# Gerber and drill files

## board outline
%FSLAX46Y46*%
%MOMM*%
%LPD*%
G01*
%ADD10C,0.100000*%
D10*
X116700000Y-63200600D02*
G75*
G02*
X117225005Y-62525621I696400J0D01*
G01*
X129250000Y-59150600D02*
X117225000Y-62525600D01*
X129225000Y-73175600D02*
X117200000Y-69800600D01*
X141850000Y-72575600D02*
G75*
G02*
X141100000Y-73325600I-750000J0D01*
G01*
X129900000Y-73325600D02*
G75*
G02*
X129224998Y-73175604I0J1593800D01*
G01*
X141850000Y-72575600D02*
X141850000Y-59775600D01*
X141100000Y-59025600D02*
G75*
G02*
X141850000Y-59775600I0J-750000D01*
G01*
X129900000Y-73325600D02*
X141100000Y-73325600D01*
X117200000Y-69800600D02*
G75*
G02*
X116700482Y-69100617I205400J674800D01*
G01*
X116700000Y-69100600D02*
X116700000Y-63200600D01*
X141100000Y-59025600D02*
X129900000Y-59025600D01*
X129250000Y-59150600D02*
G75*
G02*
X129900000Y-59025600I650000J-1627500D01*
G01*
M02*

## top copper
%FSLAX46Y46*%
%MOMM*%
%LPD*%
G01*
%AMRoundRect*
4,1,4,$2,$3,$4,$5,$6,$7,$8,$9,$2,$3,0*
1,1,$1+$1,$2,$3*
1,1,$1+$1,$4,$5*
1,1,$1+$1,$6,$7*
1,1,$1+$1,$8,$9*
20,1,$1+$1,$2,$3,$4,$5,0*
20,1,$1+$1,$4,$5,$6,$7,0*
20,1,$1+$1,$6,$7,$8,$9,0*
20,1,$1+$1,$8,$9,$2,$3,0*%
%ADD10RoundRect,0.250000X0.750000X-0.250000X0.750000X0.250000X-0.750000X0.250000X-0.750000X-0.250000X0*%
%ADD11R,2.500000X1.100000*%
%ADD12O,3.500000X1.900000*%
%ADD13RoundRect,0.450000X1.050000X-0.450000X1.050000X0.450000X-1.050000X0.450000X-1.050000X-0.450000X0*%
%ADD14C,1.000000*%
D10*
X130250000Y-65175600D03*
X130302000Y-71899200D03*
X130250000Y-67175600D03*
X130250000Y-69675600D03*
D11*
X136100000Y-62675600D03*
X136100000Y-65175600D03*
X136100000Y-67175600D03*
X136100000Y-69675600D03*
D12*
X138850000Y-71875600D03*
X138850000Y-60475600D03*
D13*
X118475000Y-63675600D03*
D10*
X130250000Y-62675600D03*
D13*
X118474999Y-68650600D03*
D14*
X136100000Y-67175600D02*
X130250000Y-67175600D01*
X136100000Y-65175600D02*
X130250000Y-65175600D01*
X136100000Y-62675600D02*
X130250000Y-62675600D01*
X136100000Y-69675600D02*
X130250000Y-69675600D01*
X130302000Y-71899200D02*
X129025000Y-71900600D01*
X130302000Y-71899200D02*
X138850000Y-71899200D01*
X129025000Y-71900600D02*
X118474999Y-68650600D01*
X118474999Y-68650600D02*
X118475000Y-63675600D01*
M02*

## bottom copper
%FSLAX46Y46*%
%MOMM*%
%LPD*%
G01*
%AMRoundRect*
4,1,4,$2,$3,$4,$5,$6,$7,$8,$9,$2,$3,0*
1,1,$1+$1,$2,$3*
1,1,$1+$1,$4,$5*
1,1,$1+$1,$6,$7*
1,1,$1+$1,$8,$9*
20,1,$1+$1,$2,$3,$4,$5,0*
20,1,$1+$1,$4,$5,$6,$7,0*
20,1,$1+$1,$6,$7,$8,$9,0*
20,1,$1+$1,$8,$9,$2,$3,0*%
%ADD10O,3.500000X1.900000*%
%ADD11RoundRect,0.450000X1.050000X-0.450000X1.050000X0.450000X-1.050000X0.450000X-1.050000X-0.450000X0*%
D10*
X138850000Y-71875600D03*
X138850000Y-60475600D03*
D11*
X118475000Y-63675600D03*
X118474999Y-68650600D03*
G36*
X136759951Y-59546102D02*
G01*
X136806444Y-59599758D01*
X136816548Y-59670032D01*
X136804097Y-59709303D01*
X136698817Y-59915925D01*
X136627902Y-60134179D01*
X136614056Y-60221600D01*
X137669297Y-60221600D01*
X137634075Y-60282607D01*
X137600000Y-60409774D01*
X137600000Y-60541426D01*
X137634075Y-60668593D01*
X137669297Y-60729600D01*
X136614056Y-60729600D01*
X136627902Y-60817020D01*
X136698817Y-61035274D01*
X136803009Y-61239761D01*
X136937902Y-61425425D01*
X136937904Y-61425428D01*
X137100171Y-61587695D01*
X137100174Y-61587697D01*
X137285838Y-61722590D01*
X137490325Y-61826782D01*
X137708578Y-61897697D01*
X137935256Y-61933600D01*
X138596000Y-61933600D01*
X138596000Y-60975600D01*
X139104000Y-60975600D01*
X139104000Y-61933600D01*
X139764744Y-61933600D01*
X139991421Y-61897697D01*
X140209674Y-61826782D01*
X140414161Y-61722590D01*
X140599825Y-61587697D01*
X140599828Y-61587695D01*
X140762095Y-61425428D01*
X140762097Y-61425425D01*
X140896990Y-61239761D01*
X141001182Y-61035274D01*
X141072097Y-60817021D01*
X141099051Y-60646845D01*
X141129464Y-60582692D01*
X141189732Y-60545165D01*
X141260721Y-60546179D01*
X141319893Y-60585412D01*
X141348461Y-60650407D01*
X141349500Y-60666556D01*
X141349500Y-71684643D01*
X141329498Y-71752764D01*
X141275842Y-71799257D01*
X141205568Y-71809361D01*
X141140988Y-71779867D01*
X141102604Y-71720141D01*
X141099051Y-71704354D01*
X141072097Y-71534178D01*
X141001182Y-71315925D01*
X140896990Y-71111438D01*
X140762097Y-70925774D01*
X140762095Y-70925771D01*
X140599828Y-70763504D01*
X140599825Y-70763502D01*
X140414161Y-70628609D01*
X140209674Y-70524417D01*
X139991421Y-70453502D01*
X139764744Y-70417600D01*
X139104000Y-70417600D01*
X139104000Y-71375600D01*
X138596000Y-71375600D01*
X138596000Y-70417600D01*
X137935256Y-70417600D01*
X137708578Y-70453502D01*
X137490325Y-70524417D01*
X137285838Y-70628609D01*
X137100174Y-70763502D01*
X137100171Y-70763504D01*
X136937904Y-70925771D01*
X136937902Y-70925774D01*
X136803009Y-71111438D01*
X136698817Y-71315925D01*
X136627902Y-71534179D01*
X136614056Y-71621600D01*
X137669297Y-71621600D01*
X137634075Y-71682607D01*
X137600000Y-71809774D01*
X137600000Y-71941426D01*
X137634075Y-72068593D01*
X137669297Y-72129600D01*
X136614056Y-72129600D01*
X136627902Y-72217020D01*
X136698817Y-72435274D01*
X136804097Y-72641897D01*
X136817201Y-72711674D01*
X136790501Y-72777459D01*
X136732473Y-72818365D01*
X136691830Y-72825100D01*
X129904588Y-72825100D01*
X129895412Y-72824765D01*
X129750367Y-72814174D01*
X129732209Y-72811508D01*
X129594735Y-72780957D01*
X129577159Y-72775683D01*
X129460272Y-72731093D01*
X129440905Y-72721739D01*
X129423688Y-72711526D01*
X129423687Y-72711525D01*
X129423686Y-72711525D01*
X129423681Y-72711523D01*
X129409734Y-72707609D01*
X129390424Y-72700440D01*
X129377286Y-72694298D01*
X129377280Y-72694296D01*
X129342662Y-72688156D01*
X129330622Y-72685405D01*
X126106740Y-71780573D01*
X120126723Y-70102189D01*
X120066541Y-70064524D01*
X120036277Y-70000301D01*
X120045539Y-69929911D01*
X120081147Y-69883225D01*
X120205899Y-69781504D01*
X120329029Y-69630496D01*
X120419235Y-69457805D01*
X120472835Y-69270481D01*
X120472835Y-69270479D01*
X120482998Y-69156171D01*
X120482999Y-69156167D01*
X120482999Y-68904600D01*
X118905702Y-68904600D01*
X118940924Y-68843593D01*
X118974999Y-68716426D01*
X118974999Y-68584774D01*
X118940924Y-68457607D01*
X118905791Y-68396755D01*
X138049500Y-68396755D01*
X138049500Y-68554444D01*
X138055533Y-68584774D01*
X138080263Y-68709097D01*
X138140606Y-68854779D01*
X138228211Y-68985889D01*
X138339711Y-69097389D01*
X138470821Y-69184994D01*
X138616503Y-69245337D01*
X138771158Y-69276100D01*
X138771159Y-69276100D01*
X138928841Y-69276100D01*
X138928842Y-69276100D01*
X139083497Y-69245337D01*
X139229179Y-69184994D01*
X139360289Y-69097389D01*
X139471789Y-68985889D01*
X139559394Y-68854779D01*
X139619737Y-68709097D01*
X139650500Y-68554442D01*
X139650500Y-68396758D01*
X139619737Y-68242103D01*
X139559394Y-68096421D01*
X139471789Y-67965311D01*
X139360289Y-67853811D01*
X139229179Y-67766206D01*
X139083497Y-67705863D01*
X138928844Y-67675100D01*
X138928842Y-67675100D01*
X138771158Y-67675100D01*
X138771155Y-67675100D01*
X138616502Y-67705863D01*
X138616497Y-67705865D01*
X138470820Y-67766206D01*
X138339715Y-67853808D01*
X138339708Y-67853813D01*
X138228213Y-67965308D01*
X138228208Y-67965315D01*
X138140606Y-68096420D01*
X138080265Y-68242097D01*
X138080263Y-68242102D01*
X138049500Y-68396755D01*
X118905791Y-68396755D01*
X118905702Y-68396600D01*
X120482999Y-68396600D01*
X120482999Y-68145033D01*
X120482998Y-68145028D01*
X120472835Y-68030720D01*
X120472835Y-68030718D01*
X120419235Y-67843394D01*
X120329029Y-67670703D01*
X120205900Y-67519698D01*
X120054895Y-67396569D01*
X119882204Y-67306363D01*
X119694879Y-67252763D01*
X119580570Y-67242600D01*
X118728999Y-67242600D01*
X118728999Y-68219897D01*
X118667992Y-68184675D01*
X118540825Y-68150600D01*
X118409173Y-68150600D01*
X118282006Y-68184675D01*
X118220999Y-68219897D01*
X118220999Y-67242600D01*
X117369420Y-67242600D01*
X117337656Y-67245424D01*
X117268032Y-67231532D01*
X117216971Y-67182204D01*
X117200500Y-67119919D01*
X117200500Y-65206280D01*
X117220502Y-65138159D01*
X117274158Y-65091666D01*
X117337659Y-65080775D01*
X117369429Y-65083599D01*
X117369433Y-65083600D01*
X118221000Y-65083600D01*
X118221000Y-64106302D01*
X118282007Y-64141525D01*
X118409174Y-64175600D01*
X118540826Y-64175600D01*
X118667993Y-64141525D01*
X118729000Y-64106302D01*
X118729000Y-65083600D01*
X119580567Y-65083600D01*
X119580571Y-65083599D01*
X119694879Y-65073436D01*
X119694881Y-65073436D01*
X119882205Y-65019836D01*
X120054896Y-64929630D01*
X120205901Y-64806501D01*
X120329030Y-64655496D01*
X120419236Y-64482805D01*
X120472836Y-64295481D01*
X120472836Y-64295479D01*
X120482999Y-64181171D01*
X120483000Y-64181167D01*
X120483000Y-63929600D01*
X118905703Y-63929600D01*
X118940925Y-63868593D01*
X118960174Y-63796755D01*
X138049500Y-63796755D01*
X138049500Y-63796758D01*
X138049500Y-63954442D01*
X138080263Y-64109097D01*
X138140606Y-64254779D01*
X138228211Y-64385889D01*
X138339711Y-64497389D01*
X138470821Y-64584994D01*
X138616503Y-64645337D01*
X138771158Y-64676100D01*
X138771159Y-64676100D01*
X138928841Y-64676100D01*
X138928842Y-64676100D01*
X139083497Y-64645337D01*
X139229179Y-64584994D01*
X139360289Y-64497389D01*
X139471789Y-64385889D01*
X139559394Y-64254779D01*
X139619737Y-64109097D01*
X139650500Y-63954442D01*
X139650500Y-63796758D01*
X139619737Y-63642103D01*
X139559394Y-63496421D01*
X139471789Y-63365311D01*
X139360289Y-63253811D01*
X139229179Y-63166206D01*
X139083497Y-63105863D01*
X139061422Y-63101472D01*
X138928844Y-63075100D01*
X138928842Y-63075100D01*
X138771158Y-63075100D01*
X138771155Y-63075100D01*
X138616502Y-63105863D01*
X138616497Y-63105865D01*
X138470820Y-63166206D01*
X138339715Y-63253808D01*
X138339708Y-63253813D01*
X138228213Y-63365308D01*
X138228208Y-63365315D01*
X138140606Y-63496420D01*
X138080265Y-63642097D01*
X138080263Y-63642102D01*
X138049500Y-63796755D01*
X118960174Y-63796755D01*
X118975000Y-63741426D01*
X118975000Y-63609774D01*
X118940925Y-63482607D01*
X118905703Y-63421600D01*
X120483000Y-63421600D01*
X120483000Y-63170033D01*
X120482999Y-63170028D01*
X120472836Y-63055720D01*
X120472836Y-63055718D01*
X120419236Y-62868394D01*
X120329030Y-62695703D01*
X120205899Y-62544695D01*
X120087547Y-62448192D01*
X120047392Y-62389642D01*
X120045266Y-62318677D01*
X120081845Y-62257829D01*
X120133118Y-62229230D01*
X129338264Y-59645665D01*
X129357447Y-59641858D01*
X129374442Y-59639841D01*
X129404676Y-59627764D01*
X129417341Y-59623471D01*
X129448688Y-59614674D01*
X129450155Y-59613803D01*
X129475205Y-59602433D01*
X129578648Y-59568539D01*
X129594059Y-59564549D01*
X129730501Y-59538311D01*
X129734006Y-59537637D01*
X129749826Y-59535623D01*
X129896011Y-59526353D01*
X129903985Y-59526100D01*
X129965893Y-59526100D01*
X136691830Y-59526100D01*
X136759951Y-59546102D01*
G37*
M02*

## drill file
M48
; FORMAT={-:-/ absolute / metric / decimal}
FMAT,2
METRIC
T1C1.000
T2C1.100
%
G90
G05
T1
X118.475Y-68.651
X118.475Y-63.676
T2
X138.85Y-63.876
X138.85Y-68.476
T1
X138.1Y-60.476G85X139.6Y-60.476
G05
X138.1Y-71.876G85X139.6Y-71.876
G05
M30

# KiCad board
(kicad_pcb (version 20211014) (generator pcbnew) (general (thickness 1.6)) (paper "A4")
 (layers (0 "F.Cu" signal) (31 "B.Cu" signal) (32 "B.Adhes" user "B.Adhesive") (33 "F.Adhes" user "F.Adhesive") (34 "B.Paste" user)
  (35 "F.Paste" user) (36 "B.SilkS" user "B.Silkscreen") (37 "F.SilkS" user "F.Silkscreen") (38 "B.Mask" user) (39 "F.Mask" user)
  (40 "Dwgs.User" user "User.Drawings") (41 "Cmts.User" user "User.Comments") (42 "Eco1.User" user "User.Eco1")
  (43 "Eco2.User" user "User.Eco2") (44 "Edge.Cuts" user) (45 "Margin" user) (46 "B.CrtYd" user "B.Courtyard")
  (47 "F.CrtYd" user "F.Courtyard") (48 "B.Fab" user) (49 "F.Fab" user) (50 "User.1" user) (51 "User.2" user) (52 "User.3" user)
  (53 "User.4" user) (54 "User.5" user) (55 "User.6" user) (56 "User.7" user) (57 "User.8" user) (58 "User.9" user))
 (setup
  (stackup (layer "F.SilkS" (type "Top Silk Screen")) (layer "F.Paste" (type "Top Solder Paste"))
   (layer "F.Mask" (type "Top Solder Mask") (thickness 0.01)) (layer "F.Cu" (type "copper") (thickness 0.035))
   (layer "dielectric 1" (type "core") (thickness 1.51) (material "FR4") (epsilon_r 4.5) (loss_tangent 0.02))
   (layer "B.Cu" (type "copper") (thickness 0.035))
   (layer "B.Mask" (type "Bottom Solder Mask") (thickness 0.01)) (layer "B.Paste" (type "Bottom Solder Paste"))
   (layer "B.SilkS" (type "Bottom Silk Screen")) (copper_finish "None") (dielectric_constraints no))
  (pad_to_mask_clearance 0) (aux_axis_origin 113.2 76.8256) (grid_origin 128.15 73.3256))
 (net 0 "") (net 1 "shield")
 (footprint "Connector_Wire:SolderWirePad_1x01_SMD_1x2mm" (layer "F.Cu") (at 130.25 65.1756 90)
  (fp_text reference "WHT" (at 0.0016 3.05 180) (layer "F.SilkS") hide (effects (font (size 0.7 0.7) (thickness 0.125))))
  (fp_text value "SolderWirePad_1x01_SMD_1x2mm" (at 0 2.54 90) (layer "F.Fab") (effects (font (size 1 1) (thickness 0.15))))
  (pad "1" smd roundrect (at 0 0 90) (size 1 2) (layers "F.Cu" "F.Paste" "F.Mask") (roundrect_rratio 0.25)))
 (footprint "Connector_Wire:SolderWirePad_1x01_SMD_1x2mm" (layer "F.Cu") (at 130.302 71.8992 90)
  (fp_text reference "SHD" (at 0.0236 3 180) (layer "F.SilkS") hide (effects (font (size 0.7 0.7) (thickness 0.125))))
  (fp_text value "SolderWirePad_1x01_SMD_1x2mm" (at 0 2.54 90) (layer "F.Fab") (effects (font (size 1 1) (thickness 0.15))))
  (pad "1" smd roundrect (at 0 0 90) (size 1 2) (layers "F.Cu" "F.Paste" "F.Mask") (roundrect_rratio 0.25)))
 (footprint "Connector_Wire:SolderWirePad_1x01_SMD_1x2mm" (layer "F.Cu") (at 130.25 67.1756 90)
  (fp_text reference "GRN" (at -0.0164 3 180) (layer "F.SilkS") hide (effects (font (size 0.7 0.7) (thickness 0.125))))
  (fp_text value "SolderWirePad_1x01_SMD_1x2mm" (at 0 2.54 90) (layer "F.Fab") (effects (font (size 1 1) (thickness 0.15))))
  (pad "1" smd roundrect (at 0 0 90) (size 1 2) (layers "F.Cu" "F.Paste" "F.Mask") (roundrect_rratio 0.25)))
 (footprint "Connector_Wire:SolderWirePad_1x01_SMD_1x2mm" (layer "F.Cu") (at 130.25 69.6756 90)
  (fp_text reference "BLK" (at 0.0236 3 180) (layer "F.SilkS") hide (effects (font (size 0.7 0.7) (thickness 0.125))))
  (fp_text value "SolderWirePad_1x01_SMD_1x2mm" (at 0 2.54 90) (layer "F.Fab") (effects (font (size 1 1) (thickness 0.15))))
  (pad "1" smd roundrect (at 0 0 90) (size 1 2) (layers "F.Cu" "F.Paste" "F.Mask") (roundrect_rratio 0.25)))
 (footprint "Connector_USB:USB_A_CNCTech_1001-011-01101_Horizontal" (layer "F.Cu") (at 145.75 66.1756)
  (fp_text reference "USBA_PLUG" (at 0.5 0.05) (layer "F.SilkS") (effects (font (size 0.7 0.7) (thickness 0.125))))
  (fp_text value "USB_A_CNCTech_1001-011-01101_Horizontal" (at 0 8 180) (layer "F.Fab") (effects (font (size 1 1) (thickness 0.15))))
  (pad "" np_thru_hole circle (at -6.9 2.3) (size 1.1 1.1) (drill 1.1) (layers *.Cu *.Mask))
  (pad "" np_thru_hole circle (at -6.9 -2.3) (size 1.1 1.1) (drill 1.1) (layers *.Cu *.Mask))
  (pad "1" smd rect (at -9.65 -3.5) (size 2.5 1.1) (layers "F.Cu" "F.Paste" "F.Mask"))
  (pad "2" smd rect (at -9.65 -1) (size 2.5 1.1) (layers "F.Cu" "F.Paste" "F.Mask"))
  (pad "3" smd rect (at -9.65 1) (size 2.5 1.1) (layers "F.Cu" "F.Paste" "F.Mask"))
  (pad "4" smd rect (at -9.65 3.5) (size 2.5 1.1) (layers "F.Cu" "F.Paste" "F.Mask"))
  (pad "5" thru_hole oval (at -6.9 5.7) (size 3.5 1.9) (drill oval 2.5 1) (layers *.Cu *.Mask) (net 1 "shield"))
  (pad "5" thru_hole oval (at -6.9 -5.7) (size 3.5 1.9) (drill oval 2.5 1) (layers *.Cu *.Mask) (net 1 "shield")))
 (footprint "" (layer "F.Cu") (at 123.375 63.4256)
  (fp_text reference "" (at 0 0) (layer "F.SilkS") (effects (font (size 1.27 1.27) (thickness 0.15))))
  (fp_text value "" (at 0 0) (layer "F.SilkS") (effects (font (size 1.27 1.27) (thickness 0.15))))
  (pad "1" thru_hole roundrect (at -4.9 0.25 90) (size 1.8 3) (drill 1) (layers *.Cu *.Mask) (roundrect_rratio 0.25) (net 1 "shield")))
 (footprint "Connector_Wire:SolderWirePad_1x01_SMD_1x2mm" (layer "F.Cu") (at 130.25 62.6756 90)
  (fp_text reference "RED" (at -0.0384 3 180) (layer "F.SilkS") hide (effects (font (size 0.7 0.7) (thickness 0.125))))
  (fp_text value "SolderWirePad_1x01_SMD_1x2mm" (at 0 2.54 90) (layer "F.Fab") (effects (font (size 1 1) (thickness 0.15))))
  (pad "1" smd roundrect (at 0 0 90) (size 1 2) (layers "F.Cu" "F.Paste" "F.Mask") (roundrect_rratio 0.25)))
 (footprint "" (layer "F.Cu") (at 118.474999 68.6506)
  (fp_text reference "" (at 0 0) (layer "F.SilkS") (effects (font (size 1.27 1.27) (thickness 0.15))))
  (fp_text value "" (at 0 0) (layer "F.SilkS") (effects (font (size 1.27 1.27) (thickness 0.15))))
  (pad "1" thru_hole roundrect (at 0 0 90) (size 1.8 3) (drill 1) (layers *.Cu *.Mask) (roundrect_rratio 0.25) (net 1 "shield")))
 (gr_arc (start 116.7 63.2006) (mid 116.846701 62.773034) (end 117.225 62.5256) (layer "Edge.Cuts") (width 0.1))
 (gr_line (start 129.25 59.1506) (end 117.225 62.5256) (layer "Edge.Cuts") (width 0.1))
 (gr_line (start 129.225 73.1756) (end 117.2 69.8006) (layer "Edge.Cuts") (width 0.1))
 (gr_arc (start 141.85 72.5756) (mid 141.63033 73.10593) (end 141.1 73.3256) (layer "Edge.Cuts") (width 0.1))
 (gr_arc (start 129.9 73.3256) (mid 129.554267 73.287648) (end 129.225 73.1756) (layer "Edge.Cuts") (width 0.1))
 (gr_line (start 141.85 72.5756) (end 141.85 59.7756) (layer "Edge.Cuts") (width 0.1))
 (gr_arc (start 141.1 59.0256) (mid 141.63033 59.24527) (end 141.85 59.7756) (layer "Edge.Cuts") (width 0.1))
 (gr_line (start 129.9 73.3256) (end 141.1 73.3256) (layer "Edge.Cuts") (width 0.1))
 (gr_arc (start 117.2 69.8006) (mid 116.831215 69.53554) (end 116.700446 69.100616) (layer "Edge.Cuts") (width 0.1))
 (gr_line (start 116.7 69.1006) (end 116.7 63.2006) (layer "Edge.Cuts") (width 0.1))
 (gr_line (start 141.1 59.0256) (end 129.9 59.0256) (layer "Edge.Cuts") (width 0.1))
 (gr_arc (start 129.25 59.1506) (mid 129.569045 59.057134) (end 129.9 59.0256) (layer "Edge.Cuts") (width 0.1))
 (segment (start 136.1 67.1756) (end 130.25 67.1756) (width 1) (layer "F.Cu") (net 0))
 (segment (start 136.1 65.1756) (end 130.25 65.1756) (width 1) (layer "F.Cu") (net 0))
 (segment (start 136.1 62.6756) (end 130.25 62.6756) (width 1) (layer "F.Cu") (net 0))
 (segment (start 136.1 69.6756) (end 130.25 69.6756) (width 1) (layer "F.Cu") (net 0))
 (segment (start 130.302 71.8992) (end 129.025 71.9006) (width 1) (layer "F.Cu") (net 1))
 (segment (start 130.302 71.8992) (end 138.85 71.8992) (width 1) (layer "F.Cu") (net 1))
 (segment (start 129.025 71.9006) (end 118.474999 68.6506) (width 1) (layer "F.Cu") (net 1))
 (segment (start 118.474999 68.6506) (end 118.475 63.6756) (width 1) (layer "F.Cu") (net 1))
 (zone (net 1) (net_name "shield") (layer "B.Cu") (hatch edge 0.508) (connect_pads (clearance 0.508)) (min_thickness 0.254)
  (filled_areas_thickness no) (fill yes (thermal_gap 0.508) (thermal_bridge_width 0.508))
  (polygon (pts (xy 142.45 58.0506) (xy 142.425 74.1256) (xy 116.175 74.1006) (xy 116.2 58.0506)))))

